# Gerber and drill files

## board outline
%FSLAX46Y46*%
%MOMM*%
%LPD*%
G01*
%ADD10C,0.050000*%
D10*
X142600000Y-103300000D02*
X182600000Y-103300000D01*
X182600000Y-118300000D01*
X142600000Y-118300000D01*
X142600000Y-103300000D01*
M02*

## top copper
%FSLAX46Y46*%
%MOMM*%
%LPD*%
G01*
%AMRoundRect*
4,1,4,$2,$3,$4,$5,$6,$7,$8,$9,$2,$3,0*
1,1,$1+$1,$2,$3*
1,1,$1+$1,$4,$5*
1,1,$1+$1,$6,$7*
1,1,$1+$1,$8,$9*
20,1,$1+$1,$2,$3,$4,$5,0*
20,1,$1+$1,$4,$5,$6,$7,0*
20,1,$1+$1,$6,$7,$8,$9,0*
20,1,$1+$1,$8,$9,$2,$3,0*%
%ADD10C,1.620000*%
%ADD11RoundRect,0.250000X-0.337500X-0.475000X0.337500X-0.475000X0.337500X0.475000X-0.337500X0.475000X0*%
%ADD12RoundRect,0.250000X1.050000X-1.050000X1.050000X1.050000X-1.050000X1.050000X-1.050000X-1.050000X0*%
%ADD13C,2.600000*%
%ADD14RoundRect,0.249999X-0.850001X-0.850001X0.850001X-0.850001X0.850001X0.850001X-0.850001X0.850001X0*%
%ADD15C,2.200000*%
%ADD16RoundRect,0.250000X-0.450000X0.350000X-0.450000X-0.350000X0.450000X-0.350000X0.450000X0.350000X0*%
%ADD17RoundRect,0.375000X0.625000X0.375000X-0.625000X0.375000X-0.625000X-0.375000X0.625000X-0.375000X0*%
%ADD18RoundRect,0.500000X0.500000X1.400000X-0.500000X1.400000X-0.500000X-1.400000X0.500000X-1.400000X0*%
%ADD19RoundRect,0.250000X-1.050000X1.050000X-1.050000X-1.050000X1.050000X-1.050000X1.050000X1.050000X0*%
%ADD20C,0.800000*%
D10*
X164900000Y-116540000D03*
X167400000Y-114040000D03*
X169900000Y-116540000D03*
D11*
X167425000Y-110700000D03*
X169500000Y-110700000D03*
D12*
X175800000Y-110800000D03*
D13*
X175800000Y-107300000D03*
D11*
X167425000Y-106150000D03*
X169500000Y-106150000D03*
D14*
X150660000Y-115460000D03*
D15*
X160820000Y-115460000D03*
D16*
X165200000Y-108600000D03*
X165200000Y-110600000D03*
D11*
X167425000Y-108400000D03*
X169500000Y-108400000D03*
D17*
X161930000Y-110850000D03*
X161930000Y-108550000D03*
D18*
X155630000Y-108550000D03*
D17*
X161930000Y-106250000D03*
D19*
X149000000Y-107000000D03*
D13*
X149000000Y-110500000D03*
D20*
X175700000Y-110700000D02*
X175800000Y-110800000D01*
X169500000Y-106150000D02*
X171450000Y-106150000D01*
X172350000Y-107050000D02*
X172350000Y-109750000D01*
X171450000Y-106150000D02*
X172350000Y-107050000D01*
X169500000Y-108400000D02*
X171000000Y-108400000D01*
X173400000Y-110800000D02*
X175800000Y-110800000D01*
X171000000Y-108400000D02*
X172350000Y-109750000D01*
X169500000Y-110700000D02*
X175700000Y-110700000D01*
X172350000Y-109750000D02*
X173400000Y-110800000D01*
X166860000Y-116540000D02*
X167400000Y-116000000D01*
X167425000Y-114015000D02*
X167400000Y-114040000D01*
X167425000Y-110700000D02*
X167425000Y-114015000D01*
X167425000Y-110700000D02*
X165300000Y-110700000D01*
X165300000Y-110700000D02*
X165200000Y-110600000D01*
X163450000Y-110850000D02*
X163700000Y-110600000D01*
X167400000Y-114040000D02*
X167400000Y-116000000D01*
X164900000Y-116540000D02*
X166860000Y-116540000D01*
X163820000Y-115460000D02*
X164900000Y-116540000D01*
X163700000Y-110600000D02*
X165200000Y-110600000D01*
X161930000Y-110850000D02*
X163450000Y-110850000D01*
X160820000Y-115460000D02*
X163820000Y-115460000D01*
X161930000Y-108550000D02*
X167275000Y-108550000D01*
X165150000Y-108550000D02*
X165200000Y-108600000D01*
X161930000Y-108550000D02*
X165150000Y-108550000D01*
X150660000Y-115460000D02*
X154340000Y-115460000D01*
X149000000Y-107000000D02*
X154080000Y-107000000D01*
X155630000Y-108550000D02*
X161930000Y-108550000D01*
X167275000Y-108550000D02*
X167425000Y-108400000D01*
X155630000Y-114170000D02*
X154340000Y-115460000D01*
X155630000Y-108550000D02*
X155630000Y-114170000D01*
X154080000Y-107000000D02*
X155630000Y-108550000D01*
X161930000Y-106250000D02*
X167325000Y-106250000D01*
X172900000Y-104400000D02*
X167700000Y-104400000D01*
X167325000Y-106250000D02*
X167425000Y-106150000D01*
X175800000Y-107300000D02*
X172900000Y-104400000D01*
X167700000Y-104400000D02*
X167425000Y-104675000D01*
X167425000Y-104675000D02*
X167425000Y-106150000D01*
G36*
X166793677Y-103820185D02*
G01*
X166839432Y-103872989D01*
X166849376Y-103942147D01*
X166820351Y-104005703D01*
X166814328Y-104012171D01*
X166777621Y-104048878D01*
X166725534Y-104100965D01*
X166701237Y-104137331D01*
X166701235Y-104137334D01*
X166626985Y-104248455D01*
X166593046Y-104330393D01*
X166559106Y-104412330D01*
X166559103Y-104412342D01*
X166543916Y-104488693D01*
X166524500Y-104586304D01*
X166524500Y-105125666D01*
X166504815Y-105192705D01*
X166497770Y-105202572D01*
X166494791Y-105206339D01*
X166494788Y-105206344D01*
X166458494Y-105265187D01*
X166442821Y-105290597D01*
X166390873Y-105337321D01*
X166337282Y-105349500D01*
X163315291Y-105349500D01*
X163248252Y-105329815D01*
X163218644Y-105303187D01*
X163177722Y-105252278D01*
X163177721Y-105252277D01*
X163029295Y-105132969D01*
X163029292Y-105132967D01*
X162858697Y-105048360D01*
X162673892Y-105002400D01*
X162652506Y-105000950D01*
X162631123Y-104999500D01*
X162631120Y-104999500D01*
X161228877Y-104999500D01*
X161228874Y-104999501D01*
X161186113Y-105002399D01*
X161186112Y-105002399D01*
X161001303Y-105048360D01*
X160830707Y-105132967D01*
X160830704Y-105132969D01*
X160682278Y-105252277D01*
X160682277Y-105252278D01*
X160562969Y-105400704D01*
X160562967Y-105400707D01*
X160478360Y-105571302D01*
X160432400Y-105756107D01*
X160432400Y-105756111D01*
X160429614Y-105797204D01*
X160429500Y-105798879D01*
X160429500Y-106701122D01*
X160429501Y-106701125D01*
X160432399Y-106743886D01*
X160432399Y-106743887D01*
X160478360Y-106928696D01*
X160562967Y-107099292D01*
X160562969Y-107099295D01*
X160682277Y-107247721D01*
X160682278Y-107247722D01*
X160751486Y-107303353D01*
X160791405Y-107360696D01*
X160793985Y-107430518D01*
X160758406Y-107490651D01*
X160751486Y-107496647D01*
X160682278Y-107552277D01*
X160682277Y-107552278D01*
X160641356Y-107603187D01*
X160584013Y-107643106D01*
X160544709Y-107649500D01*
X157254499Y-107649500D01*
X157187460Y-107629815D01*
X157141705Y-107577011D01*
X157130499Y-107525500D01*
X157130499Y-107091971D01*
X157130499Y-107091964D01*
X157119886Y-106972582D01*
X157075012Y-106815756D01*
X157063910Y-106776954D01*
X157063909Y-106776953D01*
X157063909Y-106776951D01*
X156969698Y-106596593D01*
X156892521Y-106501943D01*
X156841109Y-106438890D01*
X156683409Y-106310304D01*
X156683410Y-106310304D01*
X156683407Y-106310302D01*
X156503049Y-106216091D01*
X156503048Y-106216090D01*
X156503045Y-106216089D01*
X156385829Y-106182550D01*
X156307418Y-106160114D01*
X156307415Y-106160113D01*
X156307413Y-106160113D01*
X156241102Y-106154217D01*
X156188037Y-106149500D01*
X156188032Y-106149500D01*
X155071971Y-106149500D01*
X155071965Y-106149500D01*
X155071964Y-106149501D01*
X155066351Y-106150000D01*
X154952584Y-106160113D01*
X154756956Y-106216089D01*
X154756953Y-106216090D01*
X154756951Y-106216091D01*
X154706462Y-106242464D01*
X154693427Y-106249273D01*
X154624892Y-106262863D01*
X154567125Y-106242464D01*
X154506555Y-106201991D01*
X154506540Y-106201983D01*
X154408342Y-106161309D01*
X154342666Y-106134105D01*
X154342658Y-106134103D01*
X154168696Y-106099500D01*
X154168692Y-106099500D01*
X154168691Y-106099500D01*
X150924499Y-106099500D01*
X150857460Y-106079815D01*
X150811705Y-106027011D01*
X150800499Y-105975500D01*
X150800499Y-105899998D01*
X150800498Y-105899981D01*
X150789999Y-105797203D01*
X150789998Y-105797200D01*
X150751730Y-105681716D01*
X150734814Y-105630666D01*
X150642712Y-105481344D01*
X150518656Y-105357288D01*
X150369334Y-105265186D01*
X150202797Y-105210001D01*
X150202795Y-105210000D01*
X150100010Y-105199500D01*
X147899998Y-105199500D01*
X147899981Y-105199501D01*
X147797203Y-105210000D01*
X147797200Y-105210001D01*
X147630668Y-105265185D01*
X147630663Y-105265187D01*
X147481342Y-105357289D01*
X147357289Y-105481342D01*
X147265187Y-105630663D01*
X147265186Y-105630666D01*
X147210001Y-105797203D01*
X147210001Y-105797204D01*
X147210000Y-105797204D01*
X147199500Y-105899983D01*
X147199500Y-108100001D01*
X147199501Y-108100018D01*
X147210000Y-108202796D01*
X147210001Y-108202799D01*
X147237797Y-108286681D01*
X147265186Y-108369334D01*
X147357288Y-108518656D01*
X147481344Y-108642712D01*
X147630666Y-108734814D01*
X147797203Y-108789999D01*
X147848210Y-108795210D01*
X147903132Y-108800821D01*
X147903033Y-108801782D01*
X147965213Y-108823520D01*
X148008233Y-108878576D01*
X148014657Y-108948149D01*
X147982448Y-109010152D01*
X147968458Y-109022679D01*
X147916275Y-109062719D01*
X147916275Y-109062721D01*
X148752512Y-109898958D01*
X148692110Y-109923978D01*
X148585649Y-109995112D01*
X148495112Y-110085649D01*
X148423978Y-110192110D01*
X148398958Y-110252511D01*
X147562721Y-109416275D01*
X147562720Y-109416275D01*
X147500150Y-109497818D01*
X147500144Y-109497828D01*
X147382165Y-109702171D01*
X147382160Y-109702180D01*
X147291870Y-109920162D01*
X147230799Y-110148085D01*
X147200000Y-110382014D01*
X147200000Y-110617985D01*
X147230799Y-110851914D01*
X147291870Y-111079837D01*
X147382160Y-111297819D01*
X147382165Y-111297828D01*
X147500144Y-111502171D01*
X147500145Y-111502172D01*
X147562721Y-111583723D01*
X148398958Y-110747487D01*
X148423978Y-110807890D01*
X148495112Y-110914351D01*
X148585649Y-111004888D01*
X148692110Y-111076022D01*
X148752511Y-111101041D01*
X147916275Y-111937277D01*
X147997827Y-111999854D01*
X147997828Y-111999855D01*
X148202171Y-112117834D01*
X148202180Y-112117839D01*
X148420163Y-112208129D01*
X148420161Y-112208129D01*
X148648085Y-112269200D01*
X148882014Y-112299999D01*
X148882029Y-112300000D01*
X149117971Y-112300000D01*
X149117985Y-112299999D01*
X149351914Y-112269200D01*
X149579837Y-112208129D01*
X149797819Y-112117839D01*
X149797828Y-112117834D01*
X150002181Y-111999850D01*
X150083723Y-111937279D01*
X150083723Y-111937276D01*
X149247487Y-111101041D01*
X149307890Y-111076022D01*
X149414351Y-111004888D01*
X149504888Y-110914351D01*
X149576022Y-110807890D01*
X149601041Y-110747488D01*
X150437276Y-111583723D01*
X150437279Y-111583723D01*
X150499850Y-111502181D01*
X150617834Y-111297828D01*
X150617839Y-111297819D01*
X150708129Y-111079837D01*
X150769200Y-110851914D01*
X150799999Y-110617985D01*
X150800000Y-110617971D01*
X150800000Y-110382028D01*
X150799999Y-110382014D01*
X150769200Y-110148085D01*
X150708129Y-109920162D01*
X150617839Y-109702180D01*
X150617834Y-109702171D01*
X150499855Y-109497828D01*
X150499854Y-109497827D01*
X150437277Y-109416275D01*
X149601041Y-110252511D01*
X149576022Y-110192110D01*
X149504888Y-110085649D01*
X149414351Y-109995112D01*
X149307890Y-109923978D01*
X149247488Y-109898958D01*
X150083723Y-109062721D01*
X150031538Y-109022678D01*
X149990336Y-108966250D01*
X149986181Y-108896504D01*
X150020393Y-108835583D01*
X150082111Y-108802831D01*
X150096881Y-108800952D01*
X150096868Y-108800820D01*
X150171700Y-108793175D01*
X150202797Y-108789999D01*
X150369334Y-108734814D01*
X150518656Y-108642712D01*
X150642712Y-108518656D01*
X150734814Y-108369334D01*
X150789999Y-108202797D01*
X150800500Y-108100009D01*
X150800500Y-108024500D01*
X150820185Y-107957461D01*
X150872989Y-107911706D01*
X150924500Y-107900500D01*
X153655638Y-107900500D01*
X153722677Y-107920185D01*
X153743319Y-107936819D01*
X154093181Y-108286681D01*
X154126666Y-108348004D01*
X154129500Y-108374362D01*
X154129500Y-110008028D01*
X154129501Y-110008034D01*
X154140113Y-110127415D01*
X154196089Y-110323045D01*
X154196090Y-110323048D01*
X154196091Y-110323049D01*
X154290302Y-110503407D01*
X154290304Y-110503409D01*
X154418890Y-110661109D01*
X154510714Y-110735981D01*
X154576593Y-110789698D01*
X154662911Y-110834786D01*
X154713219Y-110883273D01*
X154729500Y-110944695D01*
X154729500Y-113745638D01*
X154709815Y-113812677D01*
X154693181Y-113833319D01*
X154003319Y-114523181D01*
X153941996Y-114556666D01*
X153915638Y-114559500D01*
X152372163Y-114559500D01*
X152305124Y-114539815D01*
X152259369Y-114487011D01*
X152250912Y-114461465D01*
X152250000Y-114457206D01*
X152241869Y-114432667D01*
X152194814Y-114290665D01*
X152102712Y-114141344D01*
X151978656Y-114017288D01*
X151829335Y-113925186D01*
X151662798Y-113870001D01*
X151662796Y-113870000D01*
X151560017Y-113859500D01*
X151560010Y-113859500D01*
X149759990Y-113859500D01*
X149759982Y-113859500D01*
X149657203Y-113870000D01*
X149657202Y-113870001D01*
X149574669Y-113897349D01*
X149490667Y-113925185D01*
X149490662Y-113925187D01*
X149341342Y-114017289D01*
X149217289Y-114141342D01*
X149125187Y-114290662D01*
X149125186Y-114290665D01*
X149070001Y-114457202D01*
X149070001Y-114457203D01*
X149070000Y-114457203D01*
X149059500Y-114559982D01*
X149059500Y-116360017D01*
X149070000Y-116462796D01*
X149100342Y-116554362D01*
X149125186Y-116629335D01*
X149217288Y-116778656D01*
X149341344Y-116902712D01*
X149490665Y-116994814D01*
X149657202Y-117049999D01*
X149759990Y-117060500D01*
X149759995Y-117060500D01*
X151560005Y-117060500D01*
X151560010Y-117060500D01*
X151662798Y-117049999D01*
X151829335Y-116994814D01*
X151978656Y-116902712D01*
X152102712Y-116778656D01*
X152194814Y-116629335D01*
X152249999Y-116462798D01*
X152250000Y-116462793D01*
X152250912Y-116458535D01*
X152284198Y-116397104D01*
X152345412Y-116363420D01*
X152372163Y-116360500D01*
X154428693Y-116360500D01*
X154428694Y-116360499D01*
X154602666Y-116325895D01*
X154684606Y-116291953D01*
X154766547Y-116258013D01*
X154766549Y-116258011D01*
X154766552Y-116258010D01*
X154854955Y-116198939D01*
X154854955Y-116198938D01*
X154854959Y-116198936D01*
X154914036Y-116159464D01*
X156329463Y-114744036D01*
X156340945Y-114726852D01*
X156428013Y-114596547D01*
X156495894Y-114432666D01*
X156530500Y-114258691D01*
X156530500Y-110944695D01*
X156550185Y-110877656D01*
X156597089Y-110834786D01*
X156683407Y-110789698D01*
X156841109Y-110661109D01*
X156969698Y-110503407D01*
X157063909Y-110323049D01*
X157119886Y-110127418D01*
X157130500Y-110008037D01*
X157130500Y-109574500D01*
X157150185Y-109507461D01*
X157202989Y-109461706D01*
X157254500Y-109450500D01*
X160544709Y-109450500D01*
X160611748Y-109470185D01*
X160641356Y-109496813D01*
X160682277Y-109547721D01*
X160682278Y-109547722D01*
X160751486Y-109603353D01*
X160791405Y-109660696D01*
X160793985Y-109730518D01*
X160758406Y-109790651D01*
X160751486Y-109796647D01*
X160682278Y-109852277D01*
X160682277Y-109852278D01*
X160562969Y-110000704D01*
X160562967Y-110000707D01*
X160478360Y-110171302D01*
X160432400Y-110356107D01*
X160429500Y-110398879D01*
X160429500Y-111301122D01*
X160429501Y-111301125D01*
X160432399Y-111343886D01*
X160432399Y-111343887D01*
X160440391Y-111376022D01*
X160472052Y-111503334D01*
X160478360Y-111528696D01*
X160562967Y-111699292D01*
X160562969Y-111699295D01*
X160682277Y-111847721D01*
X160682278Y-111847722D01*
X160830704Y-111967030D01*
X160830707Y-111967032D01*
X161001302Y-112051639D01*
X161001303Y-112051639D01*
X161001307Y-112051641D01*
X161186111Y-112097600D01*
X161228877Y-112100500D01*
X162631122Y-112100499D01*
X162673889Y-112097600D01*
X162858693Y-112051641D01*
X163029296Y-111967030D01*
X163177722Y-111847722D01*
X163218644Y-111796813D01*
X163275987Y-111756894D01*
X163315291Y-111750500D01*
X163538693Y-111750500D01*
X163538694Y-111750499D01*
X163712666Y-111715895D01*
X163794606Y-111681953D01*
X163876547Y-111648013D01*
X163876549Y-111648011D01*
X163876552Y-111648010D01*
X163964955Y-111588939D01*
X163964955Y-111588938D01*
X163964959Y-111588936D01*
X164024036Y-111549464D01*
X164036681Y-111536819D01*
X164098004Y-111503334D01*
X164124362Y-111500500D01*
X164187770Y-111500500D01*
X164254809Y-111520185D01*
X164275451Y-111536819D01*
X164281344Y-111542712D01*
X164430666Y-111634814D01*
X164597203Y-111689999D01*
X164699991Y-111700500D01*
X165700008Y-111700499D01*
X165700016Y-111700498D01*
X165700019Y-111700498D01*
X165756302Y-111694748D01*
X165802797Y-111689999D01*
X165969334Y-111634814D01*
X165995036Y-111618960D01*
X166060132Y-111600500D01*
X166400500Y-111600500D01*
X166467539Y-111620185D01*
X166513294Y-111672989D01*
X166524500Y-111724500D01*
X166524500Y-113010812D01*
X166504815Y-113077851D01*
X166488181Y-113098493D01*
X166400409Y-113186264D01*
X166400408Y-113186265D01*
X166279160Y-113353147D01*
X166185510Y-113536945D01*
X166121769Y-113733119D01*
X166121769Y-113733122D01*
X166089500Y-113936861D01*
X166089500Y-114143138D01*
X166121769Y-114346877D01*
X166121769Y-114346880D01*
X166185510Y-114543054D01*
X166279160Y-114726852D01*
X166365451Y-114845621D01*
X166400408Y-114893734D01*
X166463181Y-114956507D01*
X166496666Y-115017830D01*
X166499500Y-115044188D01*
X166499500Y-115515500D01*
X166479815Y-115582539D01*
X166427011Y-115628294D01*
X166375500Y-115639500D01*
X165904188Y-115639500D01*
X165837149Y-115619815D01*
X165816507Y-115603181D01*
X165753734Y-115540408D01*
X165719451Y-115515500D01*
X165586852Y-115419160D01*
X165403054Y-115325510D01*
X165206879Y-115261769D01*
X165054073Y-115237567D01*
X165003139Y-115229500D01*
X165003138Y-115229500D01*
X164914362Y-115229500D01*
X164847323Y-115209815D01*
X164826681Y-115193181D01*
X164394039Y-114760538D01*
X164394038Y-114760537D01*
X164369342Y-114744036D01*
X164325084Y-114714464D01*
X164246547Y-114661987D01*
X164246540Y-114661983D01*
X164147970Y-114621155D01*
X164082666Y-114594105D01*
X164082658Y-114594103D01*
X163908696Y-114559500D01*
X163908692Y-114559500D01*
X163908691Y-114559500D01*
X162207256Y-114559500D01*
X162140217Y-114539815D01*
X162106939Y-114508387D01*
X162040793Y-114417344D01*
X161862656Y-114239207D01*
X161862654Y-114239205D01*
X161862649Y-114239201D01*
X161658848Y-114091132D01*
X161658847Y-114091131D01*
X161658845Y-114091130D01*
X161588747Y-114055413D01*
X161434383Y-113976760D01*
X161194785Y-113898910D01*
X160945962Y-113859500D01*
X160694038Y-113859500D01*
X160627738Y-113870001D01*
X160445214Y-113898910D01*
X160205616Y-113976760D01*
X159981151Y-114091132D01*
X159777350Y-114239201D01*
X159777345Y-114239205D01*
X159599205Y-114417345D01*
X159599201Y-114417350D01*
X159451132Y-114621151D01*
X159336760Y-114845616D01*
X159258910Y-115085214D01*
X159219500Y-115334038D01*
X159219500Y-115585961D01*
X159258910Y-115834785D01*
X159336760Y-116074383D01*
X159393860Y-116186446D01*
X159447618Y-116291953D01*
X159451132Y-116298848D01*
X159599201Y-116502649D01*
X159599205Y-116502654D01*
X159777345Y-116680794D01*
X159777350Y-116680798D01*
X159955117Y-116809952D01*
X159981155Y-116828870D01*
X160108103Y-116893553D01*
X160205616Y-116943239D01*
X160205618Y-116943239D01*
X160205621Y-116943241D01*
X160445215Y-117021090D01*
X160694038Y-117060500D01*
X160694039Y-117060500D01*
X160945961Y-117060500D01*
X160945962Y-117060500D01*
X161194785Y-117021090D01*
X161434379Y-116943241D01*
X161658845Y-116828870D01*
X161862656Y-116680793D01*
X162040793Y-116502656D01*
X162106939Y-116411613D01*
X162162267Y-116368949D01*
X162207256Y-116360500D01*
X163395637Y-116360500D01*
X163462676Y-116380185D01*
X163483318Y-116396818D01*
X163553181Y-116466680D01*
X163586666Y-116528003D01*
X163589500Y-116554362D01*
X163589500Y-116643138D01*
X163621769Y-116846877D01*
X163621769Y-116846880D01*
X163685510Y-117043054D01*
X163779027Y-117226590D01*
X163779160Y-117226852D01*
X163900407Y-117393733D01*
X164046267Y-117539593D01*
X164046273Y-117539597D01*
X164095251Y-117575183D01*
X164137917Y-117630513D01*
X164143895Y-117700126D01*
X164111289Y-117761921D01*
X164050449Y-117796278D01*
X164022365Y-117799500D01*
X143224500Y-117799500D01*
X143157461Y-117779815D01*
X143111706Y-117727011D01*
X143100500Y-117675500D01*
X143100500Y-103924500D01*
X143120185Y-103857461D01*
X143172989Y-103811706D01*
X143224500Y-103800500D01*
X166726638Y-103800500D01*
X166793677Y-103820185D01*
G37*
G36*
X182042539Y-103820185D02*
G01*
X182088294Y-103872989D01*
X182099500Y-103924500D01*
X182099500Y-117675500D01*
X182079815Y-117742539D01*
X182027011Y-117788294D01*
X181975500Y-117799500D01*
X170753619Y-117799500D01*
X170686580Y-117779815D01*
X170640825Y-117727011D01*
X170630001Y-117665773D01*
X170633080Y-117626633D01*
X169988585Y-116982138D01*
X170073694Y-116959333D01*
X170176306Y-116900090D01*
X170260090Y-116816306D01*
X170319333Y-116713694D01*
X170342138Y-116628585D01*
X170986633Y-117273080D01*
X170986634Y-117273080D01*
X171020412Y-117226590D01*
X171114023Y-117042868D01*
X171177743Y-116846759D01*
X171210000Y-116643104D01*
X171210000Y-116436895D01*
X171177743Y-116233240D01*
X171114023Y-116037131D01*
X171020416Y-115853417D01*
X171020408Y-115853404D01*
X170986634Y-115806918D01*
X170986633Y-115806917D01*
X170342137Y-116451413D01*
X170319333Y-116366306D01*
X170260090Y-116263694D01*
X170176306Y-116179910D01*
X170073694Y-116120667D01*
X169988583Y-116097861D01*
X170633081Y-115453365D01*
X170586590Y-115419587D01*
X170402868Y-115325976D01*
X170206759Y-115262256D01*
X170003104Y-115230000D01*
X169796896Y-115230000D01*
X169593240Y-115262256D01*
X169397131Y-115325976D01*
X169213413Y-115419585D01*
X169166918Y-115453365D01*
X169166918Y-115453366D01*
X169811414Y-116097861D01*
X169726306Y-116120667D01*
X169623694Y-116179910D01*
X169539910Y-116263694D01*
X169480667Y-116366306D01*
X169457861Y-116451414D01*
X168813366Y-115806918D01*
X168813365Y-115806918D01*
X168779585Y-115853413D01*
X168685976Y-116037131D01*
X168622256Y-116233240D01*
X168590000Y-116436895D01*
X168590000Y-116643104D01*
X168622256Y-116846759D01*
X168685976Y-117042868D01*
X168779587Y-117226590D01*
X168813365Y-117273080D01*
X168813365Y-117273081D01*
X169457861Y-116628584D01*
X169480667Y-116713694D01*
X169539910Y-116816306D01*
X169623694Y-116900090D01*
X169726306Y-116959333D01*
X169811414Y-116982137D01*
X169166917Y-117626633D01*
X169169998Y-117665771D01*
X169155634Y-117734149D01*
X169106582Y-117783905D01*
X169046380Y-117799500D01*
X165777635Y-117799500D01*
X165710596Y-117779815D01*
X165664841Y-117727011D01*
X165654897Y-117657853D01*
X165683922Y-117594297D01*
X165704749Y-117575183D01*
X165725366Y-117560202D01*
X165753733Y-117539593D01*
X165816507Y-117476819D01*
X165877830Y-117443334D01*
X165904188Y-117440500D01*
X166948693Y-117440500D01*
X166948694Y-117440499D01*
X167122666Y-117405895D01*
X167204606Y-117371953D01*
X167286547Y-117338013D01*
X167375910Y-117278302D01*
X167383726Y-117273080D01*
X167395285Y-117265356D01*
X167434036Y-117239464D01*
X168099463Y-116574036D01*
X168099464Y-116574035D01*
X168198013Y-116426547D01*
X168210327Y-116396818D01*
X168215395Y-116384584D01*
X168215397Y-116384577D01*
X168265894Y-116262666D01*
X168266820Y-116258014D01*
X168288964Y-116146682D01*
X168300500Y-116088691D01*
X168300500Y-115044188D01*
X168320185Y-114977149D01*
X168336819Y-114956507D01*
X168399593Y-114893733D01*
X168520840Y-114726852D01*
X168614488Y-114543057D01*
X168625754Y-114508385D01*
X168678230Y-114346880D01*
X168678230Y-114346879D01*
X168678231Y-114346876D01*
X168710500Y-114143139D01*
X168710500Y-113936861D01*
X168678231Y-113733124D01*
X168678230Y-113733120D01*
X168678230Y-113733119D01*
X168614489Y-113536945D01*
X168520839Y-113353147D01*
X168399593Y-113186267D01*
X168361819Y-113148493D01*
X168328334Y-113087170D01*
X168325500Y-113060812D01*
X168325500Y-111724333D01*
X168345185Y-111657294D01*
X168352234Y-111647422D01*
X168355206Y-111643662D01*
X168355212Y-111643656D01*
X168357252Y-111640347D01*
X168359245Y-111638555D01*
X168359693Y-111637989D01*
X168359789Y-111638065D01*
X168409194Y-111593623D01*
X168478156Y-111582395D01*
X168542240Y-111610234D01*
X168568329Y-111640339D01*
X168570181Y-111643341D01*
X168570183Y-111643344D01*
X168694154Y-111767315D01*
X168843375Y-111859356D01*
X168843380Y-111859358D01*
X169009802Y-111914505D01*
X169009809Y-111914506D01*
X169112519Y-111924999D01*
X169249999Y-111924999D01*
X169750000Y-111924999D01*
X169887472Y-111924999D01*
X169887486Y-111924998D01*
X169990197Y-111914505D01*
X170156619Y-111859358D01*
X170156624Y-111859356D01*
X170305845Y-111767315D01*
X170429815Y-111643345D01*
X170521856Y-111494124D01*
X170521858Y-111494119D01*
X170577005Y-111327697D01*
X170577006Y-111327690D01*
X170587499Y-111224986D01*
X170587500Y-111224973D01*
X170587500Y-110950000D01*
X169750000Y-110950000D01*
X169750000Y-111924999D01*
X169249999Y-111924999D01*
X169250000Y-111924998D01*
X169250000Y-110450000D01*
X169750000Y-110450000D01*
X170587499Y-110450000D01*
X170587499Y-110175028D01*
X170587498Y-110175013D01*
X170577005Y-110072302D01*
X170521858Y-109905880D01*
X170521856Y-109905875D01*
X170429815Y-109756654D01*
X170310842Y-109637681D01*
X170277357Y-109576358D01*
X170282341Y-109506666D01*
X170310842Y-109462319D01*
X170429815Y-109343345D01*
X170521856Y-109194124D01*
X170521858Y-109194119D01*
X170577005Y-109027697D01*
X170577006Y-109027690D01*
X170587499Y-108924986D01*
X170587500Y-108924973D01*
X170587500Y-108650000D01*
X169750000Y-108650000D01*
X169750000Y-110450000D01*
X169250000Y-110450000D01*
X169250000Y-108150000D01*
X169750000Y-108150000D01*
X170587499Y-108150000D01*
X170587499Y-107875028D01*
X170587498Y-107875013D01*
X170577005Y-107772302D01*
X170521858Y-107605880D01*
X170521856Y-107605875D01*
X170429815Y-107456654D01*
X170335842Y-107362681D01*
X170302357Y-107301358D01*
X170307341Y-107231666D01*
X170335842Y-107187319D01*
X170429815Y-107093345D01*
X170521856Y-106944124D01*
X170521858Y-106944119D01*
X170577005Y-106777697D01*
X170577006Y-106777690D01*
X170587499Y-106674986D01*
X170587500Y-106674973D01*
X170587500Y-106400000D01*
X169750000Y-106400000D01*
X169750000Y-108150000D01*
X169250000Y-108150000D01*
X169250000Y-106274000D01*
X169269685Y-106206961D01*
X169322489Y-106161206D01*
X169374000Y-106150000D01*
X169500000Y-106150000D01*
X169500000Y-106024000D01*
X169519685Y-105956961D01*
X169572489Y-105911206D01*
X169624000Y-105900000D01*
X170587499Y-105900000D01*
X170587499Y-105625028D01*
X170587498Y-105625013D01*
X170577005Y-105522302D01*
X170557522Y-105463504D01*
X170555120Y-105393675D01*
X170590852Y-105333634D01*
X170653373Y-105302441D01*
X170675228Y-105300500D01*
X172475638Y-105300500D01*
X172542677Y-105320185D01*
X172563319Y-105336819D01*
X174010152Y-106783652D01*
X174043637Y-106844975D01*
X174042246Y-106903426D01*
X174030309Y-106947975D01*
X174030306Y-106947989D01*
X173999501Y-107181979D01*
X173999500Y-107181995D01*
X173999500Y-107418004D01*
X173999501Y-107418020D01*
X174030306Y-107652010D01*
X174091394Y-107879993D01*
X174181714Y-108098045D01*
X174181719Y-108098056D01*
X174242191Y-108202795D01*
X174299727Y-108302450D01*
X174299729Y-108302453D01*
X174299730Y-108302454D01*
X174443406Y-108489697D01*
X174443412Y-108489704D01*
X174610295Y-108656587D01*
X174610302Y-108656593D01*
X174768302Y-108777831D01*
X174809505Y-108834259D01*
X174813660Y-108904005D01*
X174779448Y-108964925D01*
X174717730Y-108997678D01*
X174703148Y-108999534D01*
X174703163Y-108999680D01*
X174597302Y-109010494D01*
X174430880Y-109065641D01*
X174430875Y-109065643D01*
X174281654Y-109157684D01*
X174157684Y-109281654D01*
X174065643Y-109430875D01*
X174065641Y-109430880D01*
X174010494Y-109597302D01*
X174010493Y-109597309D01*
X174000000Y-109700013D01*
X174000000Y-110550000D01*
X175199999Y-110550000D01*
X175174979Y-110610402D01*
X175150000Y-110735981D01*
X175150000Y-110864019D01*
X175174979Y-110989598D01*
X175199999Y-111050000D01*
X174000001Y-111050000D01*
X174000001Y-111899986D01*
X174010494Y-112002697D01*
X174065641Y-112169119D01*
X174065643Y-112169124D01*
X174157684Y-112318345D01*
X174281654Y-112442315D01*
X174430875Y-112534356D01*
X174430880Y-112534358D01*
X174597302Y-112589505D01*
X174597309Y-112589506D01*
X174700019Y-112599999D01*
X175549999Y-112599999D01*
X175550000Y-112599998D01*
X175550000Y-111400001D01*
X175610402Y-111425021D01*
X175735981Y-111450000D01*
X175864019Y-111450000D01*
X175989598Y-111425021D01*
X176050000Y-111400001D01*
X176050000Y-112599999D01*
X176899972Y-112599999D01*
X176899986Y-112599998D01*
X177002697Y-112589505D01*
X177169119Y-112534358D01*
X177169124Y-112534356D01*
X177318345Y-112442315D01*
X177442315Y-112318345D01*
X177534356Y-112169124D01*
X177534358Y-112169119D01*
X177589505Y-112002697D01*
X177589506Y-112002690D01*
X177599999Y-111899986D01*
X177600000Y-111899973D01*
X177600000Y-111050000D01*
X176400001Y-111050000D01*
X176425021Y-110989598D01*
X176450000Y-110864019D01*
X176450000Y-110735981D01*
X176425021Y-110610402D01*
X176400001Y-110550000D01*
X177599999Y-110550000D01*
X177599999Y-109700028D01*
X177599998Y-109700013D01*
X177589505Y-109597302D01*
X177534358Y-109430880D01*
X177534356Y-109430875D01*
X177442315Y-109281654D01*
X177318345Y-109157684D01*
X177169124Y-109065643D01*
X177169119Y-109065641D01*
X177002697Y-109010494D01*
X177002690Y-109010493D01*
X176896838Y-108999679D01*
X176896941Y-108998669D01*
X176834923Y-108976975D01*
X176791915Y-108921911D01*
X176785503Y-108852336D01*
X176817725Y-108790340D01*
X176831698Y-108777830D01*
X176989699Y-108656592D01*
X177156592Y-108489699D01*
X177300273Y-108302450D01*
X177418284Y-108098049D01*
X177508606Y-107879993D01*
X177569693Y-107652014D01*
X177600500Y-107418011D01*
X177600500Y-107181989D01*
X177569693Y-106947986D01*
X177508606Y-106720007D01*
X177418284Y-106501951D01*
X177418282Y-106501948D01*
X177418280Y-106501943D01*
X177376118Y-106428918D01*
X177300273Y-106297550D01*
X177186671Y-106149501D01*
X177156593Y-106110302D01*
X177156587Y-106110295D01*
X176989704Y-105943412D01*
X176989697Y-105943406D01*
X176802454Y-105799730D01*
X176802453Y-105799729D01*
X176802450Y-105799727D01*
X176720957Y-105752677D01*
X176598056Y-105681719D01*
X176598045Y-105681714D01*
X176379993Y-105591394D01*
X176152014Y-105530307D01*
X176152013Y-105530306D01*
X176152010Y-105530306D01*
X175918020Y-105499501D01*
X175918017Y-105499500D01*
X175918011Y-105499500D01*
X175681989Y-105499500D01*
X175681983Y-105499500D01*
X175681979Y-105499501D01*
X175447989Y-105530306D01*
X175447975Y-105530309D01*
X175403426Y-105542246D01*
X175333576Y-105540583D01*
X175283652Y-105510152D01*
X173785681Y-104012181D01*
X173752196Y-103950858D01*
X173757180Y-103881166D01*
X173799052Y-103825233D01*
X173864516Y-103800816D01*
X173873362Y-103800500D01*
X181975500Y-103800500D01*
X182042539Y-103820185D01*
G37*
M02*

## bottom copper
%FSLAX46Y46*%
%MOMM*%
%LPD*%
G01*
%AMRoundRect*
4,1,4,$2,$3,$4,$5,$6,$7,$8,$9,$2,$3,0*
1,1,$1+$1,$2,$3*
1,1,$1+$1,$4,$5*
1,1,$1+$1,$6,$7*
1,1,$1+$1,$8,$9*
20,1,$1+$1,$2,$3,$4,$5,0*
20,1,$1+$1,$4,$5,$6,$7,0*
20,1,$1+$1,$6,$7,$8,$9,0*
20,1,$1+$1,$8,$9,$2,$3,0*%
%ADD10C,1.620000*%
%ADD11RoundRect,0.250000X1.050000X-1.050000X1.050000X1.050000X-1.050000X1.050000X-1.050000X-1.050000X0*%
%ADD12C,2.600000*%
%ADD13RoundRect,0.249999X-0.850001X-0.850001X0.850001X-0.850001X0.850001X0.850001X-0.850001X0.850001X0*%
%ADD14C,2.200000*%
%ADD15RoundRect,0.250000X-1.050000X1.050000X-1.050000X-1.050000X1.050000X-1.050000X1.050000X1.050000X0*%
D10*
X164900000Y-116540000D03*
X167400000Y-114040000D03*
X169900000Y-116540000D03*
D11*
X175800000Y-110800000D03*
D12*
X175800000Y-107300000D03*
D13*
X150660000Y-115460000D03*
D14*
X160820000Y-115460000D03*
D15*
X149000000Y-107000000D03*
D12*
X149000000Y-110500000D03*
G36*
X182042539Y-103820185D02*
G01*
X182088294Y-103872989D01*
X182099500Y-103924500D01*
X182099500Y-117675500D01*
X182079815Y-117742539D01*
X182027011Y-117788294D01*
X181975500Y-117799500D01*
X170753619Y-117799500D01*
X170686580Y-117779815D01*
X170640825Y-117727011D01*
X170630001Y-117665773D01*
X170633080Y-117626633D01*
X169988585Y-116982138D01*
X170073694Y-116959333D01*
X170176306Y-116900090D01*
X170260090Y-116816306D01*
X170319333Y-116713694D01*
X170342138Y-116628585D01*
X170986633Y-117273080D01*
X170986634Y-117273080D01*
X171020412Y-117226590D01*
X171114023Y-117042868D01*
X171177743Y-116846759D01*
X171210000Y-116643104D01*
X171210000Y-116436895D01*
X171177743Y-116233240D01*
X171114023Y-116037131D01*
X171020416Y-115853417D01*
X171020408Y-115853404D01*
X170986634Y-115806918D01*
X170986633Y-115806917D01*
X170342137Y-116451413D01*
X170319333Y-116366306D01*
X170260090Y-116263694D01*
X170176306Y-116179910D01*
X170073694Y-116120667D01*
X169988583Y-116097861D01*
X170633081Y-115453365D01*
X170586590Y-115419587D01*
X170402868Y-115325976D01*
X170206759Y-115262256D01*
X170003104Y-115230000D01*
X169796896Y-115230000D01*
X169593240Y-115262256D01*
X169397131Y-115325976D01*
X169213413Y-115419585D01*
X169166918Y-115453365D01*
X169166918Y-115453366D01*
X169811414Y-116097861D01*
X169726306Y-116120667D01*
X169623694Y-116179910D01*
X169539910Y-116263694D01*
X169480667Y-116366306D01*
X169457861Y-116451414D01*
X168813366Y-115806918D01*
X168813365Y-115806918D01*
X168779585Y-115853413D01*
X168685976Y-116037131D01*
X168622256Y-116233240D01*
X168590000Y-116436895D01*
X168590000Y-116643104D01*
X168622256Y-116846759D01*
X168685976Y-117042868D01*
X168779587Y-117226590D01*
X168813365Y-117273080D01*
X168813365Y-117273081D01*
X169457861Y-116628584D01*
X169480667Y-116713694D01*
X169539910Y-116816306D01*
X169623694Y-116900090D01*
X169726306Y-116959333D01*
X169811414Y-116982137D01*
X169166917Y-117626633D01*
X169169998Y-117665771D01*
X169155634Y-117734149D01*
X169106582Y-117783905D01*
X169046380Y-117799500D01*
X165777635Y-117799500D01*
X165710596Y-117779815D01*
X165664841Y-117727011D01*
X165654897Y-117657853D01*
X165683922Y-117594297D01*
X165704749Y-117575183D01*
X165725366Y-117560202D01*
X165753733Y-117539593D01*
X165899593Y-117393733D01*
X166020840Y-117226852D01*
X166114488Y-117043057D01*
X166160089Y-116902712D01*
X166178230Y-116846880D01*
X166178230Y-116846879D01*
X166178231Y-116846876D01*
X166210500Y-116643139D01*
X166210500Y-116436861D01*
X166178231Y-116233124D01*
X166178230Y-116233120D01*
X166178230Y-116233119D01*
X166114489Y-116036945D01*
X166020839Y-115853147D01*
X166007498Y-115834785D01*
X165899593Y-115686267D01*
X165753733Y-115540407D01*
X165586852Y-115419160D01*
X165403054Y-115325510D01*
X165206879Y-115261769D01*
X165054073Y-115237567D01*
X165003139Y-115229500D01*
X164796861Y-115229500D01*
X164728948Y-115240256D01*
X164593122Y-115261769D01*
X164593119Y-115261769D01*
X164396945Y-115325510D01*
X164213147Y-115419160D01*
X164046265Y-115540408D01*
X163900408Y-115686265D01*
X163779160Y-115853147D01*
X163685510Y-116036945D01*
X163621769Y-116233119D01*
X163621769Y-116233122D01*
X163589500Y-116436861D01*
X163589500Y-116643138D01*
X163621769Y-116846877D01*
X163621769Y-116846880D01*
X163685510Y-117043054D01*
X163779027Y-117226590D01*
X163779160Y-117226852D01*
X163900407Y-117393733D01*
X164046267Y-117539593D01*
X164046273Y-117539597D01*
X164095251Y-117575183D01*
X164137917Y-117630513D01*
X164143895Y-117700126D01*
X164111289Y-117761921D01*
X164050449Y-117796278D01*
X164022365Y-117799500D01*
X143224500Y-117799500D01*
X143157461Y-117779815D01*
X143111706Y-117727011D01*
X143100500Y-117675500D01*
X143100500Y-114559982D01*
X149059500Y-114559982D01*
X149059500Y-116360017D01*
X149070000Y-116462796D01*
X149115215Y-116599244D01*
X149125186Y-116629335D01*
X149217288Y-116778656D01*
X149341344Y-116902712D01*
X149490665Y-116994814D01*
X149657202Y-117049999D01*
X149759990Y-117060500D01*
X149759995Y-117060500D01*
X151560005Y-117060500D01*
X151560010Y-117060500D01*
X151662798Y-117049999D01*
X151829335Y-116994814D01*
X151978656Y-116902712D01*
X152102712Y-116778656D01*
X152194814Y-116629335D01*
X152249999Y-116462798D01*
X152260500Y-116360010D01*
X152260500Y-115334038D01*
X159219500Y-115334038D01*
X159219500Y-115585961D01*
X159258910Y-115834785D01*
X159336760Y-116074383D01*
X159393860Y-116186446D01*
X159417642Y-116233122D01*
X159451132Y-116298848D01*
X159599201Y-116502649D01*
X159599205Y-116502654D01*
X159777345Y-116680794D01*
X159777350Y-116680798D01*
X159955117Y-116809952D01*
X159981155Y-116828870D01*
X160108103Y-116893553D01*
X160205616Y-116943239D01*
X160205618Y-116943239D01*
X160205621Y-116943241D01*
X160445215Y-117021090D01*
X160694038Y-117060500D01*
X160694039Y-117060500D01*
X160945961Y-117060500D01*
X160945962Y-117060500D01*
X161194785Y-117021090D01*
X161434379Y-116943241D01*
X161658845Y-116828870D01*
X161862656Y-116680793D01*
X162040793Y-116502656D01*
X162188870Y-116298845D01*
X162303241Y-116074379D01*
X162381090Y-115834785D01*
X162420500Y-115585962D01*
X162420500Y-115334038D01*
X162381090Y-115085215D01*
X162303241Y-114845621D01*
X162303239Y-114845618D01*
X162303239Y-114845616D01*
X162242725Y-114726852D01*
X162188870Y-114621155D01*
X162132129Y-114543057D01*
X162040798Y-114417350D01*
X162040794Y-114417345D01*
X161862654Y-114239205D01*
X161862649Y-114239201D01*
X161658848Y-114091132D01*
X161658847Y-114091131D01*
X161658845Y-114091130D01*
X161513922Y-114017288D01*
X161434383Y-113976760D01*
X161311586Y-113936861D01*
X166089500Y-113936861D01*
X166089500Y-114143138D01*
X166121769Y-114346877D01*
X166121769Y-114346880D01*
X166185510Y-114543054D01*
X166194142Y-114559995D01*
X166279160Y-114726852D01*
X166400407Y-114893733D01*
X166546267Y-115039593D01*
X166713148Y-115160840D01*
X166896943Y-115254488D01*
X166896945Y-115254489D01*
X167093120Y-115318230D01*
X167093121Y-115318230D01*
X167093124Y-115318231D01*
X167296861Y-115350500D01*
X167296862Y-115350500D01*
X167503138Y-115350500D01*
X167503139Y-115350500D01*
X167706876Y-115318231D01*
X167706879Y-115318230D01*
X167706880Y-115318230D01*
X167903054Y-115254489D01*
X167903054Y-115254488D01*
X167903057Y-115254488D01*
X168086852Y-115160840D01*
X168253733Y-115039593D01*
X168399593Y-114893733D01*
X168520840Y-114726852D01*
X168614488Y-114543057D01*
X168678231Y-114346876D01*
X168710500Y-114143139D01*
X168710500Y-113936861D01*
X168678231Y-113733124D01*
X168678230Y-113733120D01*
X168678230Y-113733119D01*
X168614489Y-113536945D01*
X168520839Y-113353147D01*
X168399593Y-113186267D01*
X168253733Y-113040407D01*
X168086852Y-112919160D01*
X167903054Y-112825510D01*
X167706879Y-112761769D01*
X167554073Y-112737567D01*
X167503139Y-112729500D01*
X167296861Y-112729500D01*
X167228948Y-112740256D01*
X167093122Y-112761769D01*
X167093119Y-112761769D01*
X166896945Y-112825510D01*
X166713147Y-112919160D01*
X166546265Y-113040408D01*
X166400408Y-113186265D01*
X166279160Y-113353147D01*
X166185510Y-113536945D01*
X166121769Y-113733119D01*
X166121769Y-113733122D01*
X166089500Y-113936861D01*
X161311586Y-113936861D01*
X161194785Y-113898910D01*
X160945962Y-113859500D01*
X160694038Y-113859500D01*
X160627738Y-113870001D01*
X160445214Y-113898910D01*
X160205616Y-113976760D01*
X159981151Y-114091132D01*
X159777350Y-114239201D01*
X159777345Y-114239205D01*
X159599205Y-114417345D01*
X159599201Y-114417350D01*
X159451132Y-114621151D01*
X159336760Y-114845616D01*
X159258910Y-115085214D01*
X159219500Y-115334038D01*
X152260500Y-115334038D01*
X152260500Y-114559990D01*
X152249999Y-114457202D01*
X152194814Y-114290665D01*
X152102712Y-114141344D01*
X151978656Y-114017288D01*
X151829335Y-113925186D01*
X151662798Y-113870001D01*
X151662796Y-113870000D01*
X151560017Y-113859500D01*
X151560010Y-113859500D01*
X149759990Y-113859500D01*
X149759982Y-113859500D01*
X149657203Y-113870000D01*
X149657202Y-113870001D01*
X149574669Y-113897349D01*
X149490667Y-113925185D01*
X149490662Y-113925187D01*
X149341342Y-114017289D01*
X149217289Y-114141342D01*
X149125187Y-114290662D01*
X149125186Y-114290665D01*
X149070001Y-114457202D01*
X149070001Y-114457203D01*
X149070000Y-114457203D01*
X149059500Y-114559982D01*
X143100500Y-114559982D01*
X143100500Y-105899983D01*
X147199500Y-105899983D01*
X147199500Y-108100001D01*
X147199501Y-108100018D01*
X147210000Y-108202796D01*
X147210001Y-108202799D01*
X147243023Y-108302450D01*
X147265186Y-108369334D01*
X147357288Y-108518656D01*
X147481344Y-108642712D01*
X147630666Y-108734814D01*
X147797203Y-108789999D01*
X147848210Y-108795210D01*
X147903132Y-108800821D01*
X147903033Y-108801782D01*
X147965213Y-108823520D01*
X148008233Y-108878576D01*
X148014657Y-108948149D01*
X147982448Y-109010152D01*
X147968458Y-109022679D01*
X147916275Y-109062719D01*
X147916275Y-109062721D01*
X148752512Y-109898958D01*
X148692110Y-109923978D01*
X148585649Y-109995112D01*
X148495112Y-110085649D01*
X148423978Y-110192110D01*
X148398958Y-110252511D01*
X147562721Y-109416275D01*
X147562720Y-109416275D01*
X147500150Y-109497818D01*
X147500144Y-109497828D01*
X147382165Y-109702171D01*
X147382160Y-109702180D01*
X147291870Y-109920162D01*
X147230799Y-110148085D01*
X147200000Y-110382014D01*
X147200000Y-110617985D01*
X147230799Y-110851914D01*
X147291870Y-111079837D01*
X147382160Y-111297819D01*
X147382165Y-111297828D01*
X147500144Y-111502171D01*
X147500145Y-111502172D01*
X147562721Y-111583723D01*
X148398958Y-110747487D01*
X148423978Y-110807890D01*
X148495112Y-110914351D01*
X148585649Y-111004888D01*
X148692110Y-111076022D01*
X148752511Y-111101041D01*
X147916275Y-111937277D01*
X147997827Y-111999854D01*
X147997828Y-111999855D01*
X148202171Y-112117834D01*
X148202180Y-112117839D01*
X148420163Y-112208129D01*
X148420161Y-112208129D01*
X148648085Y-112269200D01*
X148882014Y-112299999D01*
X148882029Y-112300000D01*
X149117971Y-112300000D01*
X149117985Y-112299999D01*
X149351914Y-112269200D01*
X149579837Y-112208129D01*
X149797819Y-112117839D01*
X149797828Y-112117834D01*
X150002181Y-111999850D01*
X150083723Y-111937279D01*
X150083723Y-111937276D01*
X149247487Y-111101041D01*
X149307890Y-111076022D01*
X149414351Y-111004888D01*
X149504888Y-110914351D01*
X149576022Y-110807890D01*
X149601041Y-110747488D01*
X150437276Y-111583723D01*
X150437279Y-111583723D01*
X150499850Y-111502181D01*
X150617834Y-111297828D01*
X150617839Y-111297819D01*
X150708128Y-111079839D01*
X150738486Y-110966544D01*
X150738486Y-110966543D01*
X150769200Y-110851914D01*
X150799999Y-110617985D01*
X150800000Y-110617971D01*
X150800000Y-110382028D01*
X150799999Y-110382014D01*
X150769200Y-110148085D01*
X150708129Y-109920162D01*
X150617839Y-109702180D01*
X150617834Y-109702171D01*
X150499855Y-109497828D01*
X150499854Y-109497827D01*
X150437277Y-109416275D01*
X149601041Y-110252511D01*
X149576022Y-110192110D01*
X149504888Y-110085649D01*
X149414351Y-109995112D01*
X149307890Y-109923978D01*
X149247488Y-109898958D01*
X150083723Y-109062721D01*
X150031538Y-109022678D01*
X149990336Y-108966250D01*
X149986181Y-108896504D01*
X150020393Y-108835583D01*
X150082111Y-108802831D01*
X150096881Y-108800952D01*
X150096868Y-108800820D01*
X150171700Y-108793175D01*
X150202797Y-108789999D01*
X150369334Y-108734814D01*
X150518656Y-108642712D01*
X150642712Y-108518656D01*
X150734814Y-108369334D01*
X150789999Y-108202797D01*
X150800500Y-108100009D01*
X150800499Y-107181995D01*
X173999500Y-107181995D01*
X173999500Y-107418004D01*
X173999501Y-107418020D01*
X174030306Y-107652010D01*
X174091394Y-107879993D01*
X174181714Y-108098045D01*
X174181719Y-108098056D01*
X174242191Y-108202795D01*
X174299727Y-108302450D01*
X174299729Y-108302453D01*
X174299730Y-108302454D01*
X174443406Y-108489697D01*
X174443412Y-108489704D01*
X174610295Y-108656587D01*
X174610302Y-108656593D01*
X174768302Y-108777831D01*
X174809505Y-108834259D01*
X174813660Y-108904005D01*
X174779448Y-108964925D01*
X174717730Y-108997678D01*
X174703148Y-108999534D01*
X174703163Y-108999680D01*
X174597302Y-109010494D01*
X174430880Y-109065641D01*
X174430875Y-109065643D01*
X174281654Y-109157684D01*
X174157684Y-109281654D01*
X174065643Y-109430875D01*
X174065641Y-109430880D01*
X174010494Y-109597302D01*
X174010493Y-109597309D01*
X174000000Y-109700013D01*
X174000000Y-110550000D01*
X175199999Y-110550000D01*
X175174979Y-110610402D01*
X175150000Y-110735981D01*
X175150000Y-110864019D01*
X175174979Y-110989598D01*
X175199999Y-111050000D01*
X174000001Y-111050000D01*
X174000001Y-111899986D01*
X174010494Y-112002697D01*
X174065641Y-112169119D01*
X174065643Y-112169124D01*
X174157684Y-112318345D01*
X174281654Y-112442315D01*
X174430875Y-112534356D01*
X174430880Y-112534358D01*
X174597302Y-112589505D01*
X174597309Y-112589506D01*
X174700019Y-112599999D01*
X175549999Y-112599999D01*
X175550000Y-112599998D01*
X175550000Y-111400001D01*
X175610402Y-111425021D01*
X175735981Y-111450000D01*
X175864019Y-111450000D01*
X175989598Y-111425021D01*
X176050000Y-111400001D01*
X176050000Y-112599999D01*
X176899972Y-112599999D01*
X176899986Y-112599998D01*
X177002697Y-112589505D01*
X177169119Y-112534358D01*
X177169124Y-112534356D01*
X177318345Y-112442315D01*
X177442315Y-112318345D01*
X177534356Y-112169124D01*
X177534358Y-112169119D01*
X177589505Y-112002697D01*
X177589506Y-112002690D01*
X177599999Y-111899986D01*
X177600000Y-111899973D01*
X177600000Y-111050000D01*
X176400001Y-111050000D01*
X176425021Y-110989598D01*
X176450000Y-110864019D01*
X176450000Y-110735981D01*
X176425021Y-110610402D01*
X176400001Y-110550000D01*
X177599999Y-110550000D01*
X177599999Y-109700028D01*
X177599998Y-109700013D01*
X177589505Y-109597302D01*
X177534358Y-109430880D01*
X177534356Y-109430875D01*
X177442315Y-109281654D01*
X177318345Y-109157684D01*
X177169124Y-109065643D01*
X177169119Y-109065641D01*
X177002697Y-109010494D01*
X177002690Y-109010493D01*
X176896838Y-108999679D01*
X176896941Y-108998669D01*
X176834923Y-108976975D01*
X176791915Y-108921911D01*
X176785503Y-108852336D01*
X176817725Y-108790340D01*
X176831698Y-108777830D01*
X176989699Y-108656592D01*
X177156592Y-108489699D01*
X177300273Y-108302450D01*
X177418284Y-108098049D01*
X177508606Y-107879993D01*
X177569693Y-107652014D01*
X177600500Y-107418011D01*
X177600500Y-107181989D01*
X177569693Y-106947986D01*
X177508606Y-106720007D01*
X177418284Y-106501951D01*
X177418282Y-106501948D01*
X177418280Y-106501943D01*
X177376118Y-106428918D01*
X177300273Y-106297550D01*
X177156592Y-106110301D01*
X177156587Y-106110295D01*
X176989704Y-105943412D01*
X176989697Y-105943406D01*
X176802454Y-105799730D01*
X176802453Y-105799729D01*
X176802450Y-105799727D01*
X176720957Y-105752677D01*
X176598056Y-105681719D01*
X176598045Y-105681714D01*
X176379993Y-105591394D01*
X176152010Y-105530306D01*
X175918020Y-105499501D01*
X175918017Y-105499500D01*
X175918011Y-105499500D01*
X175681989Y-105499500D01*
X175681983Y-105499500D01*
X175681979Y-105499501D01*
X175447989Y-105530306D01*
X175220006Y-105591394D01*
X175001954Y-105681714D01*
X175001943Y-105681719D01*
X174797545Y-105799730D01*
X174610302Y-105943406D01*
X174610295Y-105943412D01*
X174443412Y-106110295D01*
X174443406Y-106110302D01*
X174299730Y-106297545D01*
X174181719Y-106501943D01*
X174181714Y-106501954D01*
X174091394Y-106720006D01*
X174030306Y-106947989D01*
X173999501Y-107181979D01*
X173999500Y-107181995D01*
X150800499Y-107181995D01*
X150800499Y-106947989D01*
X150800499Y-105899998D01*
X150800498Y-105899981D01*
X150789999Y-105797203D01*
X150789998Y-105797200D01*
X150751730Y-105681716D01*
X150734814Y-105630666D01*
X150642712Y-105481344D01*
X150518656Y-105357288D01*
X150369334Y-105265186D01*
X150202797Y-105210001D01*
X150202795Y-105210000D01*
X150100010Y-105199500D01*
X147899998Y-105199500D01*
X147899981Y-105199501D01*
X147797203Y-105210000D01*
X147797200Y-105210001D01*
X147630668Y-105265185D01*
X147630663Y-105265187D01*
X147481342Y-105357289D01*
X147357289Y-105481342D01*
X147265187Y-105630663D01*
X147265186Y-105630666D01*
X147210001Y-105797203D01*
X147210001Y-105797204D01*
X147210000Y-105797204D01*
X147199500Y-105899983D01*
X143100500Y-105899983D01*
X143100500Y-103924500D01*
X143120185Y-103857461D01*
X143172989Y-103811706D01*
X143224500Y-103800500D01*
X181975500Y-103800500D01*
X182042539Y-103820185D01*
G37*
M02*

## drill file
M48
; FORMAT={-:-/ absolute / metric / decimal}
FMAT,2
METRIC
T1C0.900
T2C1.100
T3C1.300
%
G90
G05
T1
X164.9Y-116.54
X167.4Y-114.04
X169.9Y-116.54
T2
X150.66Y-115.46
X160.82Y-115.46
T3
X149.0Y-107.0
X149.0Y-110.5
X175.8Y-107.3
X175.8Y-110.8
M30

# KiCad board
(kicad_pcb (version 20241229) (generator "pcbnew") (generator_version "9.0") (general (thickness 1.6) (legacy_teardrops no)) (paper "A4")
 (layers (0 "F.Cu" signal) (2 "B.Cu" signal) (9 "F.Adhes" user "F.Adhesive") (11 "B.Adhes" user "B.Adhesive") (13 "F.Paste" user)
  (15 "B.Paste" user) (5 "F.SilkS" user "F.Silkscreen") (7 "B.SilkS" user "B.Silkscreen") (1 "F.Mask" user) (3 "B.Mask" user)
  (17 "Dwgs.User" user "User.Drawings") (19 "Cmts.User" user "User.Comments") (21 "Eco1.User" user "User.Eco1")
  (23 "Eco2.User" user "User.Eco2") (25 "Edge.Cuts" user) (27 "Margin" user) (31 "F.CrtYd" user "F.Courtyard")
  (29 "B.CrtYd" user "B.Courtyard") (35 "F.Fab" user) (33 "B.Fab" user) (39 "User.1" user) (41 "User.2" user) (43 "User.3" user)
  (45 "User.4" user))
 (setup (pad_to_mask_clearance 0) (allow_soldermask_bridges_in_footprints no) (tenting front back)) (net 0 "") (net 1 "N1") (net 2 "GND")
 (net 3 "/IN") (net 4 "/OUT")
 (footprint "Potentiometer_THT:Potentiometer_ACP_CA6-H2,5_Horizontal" (layer "F.Cu") (at 164.9 116.54 90)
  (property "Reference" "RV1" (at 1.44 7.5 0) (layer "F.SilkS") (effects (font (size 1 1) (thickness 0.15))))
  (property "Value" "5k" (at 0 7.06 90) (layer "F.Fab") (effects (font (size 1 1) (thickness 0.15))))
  (pad "1" thru_hole circle (at 0 0 90) (size 1.62 1.62) (drill 0.9) (layers "*.Cu" "*.Mask") (remove_unused_layers no) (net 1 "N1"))
  (pad "2" thru_hole circle (at 2.5 2.5 90) (size 1.62 1.62) (drill 0.9) (layers "*.Cu" "*.Mask") (remove_unused_layers no) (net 1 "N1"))
  (pad "3" thru_hole circle (at 0 5 90) (size 1.62 1.62) (drill 0.9) (layers "*.Cu" "*.Mask") (remove_unused_layers no) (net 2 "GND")))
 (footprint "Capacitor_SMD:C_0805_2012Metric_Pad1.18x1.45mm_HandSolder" (layer "F.Cu") (at 168.4625 110.7)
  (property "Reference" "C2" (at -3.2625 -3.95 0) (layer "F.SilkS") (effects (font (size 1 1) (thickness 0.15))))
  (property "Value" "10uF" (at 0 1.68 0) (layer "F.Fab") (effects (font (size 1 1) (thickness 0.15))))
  (pad "1" smd roundrect (at -1.0375 0) (size 1.175 1.45) (layers "F.Cu" "F.Mask" "F.Paste") (roundrect_rratio 0.212766) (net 1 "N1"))
  (pad "2" smd roundrect (at 1.0375 0) (size 1.175 1.45) (layers "F.Cu" "F.Mask" "F.Paste") (roundrect_rratio 0.212766) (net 2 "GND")))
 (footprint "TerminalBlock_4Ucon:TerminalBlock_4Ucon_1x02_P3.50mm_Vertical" (layer "F.Cu") (at 175.8 110.8 90)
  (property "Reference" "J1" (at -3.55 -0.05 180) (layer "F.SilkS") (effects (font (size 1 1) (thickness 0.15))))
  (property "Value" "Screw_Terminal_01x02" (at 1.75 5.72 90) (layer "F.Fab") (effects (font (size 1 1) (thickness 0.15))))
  (pad "1" thru_hole roundrect (at 0 0 90) (size 2.6 2.6) (drill 1.3) (layers "*.Cu" "*.Mask") (remove_unused_layers no)
   (roundrect_rratio 0.096154) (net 2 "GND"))
  (pad "2" thru_hole circle (at 3.5 0 90) (size 2.6 2.6) (drill 1.3) (layers "*.Cu" "*.Mask") (remove_unused_layers no) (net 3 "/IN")))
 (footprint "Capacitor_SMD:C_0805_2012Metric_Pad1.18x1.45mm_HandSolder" (layer "F.Cu") (at 168.4625 106.15)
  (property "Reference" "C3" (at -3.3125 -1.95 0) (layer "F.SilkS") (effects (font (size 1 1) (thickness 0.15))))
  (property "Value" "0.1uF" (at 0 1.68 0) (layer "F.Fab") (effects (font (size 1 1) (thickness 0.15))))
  (pad "1" smd roundrect (at -1.0375 0) (size 1.175 1.45) (layers "F.Cu" "F.Mask" "F.Paste") (roundrect_rratio 0.212766) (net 3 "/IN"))
  (pad "2" smd roundrect (at 1.0375 0) (size 1.175 1.45) (layers "F.Cu" "F.Mask" "F.Paste") (roundrect_rratio 0.212766) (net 2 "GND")))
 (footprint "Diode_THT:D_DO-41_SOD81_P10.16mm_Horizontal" (layer "F.Cu") (at 150.66 115.46)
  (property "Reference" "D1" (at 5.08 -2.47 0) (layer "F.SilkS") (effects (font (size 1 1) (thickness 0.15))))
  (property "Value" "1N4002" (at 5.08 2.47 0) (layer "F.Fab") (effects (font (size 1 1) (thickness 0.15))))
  (pad "1" thru_hole roundrect (at 0 0) (size 2.2 2.2) (drill 1.1) (layers "*.Cu" "*.Mask") (remove_unused_layers no)
   (roundrect_rratio 0.113636) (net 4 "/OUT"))
  (pad "2" thru_hole circle (at 10.16 0) (size 2.2 2.2) (drill 1.1) (layers "*.Cu" "*.Mask") (remove_unused_layers no) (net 1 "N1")))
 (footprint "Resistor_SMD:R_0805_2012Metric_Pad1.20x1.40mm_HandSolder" (layer "F.Cu") (at 165.2 109.6 -90)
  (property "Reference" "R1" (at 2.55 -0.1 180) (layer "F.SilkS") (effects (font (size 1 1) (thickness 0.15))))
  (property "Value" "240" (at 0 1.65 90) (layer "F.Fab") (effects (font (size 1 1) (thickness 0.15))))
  (pad "1" smd roundrect (at -1 0 270) (size 1.2 1.4) (layers "F.Cu" "F.Mask" "F.Paste") (roundrect_rratio 0.208333) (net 4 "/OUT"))
  (pad "2" smd roundrect (at 1 0 270) (size 1.2 1.4) (layers "F.Cu" "F.Mask" "F.Paste") (roundrect_rratio 0.208333) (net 1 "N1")))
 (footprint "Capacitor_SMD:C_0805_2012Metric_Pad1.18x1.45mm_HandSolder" (layer "F.Cu") (at 168.4625 108.4)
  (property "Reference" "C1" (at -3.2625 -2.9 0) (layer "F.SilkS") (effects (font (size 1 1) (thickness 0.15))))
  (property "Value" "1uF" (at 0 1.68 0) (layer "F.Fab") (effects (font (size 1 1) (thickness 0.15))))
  (pad "1" smd roundrect (at -1.0375 0) (size 1.175 1.45) (layers "F.Cu" "F.Mask" "F.Paste") (roundrect_rratio 0.212766) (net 4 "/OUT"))
  (pad "2" smd roundrect (at 1.0375 0) (size 1.175 1.45) (layers "F.Cu" "F.Mask" "F.Paste") (roundrect_rratio 0.212766) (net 2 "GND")))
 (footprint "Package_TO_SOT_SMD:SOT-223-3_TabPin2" (layer "F.Cu") (at 158.78 108.55 180)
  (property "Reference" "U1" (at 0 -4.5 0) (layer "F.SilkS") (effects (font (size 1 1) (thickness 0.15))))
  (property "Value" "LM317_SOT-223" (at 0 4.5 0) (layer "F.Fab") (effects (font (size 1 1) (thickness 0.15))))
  (pad "1" smd roundrect (at -3.15 -2.3 180) (size 2 1.5) (layers "F.Cu" "F.Mask" "F.Paste") (roundrect_rratio 0.25) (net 1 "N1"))
  (pad "2" smd roundrect (at -3.15 0 180) (size 2 1.5) (layers "F.Cu" "F.Mask" "F.Paste") (roundrect_rratio 0.25) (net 4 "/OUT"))
  (pad "2" smd roundrect (at 3.15 0 180) (size 2 3.8) (layers "F.Cu" "F.Mask" "F.Paste") (roundrect_rratio 0.25) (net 4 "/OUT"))
  (pad "3" smd roundrect (at -3.15 2.3 180) (size 2 1.5) (layers "F.Cu" "F.Mask" "F.Paste") (roundrect_rratio 0.25) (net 3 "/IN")))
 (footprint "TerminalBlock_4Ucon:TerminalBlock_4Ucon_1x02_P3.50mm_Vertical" (layer "F.Cu") (at 149 107 -90)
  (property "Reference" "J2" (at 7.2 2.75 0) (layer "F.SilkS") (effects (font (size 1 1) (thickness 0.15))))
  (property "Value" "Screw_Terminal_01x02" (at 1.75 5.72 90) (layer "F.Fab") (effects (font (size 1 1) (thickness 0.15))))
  (pad "1" thru_hole roundrect (at 0 0 270) (size 2.6 2.6) (drill 1.3) (layers "*.Cu" "*.Mask") (remove_unused_layers no)
   (roundrect_rratio 0.096154) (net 4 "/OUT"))
  (pad "2" thru_hole circle (at 3.5 0 270) (size 2.6 2.6) (drill 1.3) (layers "*.Cu" "*.Mask") (remove_unused_layers no) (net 2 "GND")))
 (gr_rect (start 142.6 103.3) (end 182.6 118.3) (stroke (width 0.05) (type solid)) (fill no) (layer "Edge.Cuts"))
 (segment (start 175.7 110.7) (end 175.8 110.8) (width 0.8) (layer "F.Cu") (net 2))
 (segment (start 169.5 106.15) (end 171.45 106.15) (width 0.8) (layer "F.Cu") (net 2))
 (segment (start 172.35 107.05) (end 172.35 109.75) (width 0.8) (layer "F.Cu") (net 2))
 (segment (start 171.45 106.15) (end 172.35 107.05) (width 0.8) (layer "F.Cu") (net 2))
 (segment (start 169.5 108.4) (end 171 108.4) (width 0.8) (layer "F.Cu") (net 2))
 (segment (start 173.4 110.8) (end 175.8 110.8) (width 0.8) (layer "F.Cu") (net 2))
 (segment (start 171 108.4) (end 172.35 109.75) (width 0.8) (layer "F.Cu") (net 2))
 (segment (start 169.5 110.7) (end 175.7 110.7) (width 0.8) (layer "F.Cu") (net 2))
 (segment (start 172.35 109.75) (end 173.4 110.8) (width 0.8) (layer "F.Cu") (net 2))
 (segment (start 166.86 116.54) (end 167.4 116) (width 0.8) (layer "F.Cu") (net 1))
 (segment (start 167.425 114.015) (end 167.4 114.04) (width 0.8) (layer "F.Cu") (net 1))
 (segment (start 167.425 110.7) (end 167.425 114.015) (width 0.8) (layer "F.Cu") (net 1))
 (segment (start 167.425 110.7) (end 165.3 110.7) (width 0.8) (layer "F.Cu") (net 1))
 (segment (start 165.3 110.7) (end 165.2 110.6) (width 0.8) (layer "F.Cu") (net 1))
 (segment (start 163.45 110.85) (end 163.7 110.6) (width 0.8) (layer "F.Cu") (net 1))
 (segment (start 167.4 114.04) (end 167.4 116) (width 0.8) (layer "F.Cu") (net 1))
 (segment (start 164.9 116.54) (end 166.86 116.54) (width 0.8) (layer "F.Cu") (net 1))
 (segment (start 163.82 115.46) (end 164.9 116.54) (width 0.8) (layer "F.Cu") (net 1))
 (segment (start 163.7 110.6) (end 165.2 110.6) (width 0.8) (layer "F.Cu") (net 1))
 (segment (start 161.93 110.85) (end 163.45 110.85) (width 0.8) (layer "F.Cu") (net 1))
 (segment (start 160.82 115.46) (end 163.82 115.46) (width 0.8) (layer "F.Cu") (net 1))
 (segment (start 161.93 108.55) (end 167.275 108.55) (width 0.8) (layer "F.Cu") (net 4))
 (segment (start 165.15 108.55) (end 165.2 108.6) (width 0.8) (layer "F.Cu") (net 4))
 (segment (start 161.93 108.55) (end 165.15 108.55) (width 0.8) (layer "F.Cu") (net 4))
 (segment (start 150.66 115.46) (end 154.34 115.46) (width 0.8) (layer "F.Cu") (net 4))
 (segment (start 149 107) (end 154.08 107) (width 0.8) (layer "F.Cu") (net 4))
 (segment (start 155.63 108.55) (end 161.93 108.55) (width 0.8) (layer "F.Cu") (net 4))
 (segment (start 167.275 108.55) (end 167.425 108.4) (width 0.8) (layer "F.Cu") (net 4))
 (segment (start 155.63 114.17) (end 154.34 115.46) (width 0.8) (layer "F.Cu") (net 4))
 (segment (start 155.63 108.55) (end 155.63 114.17) (width 0.8) (layer "F.Cu") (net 4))
 (segment (start 154.08 107) (end 155.63 108.55) (width 0.8) (layer "F.Cu") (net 4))
 (segment (start 161.93 106.25) (end 167.325 106.25) (width 0.8) (layer "F.Cu") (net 3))
 (segment (start 172.9 104.4) (end 167.7 104.4) (width 0.8) (layer "F.Cu") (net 3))
 (segment (start 167.325 106.25) (end 167.425 106.15) (width 0.8) (layer "F.Cu") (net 3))
 (segment (start 175.8 107.3) (end 172.9 104.4) (width 0.8) (layer "F.Cu") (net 3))
 (segment (start 167.7 104.4) (end 167.425 104.675) (width 0.8) (layer "F.Cu") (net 3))
 (segment (start 167.425 104.675) (end 167.425 106.15) (width 0.8) (layer "F.Cu") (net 3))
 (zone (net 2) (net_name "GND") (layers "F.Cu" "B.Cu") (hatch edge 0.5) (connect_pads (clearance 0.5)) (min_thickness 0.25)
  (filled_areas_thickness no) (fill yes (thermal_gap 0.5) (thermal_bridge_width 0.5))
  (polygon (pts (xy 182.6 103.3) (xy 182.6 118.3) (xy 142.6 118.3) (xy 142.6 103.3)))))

